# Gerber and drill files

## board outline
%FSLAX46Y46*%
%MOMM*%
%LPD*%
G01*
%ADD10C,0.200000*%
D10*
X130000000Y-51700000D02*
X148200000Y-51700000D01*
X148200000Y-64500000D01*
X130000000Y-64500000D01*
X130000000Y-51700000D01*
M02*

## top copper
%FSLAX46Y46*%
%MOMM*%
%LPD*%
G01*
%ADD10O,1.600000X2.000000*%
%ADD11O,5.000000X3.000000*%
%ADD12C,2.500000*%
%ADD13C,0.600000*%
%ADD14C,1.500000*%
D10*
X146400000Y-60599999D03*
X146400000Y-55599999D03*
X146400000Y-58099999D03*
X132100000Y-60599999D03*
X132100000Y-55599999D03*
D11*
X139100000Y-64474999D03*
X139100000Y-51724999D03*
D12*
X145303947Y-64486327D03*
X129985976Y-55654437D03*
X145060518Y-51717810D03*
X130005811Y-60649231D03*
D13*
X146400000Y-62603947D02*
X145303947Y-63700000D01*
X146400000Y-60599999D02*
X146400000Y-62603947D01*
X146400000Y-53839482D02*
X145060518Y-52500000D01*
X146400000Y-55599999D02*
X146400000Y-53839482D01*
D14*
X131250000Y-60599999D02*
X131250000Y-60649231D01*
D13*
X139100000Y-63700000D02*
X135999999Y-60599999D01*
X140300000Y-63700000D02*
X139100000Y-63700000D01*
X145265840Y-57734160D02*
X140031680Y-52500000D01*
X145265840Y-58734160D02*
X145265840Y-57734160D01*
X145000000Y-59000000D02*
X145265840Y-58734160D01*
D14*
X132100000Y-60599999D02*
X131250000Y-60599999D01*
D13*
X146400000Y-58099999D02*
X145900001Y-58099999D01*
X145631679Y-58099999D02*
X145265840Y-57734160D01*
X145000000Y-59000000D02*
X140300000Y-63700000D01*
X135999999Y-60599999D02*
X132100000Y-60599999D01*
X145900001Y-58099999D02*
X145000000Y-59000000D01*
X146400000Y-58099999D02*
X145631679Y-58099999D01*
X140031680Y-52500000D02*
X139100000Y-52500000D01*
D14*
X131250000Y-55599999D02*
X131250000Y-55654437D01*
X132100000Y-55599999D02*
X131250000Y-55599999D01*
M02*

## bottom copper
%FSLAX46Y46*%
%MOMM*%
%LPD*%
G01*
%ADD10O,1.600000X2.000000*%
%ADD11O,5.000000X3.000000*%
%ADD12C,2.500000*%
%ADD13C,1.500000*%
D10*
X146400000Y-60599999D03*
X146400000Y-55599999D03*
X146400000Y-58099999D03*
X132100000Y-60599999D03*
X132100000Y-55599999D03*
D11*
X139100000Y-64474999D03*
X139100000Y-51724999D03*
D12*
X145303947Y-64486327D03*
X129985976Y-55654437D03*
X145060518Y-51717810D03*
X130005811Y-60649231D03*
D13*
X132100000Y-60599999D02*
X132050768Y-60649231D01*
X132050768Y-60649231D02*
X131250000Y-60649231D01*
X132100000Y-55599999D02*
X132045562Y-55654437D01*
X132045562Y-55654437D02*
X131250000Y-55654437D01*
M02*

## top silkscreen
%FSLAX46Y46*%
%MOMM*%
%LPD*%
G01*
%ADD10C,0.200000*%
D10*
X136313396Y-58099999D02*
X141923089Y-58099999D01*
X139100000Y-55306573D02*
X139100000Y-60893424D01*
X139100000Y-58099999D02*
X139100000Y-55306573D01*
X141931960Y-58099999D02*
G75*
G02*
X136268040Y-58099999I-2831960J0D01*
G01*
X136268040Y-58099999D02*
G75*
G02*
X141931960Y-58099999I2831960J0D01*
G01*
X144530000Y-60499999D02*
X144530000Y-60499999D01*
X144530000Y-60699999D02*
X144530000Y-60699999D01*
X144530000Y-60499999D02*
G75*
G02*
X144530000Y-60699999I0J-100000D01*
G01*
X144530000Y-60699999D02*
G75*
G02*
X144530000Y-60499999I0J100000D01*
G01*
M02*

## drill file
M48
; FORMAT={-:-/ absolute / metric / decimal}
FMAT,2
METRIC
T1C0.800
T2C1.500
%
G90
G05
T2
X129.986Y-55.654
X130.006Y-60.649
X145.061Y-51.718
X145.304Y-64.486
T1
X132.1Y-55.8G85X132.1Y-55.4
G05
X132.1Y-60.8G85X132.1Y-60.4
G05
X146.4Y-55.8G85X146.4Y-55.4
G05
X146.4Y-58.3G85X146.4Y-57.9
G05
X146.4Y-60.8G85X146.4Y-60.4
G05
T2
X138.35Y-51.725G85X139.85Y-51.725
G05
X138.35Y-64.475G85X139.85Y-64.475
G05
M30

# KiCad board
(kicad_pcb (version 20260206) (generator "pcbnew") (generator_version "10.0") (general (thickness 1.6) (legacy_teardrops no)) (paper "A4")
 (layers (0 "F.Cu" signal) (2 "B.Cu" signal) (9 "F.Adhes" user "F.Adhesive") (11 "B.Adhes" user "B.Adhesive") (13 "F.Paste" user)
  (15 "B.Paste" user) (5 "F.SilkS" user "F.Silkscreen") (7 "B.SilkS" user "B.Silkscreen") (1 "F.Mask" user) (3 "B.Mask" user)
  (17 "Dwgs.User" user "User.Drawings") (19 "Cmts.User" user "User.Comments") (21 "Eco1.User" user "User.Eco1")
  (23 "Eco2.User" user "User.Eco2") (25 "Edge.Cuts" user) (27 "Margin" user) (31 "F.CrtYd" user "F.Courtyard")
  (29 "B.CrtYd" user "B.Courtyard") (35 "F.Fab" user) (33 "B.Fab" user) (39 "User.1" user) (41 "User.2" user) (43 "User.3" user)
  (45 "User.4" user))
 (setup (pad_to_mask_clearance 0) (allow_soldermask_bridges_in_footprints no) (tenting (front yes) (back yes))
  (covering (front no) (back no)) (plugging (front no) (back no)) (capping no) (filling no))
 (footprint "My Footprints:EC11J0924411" (layer "F.Cu") (at 139.1 58.099999 90)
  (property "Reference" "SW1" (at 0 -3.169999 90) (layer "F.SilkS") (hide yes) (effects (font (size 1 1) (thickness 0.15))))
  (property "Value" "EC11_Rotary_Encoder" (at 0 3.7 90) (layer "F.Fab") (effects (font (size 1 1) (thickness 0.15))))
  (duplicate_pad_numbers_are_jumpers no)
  (fp_line (start -2.4 5.43) (end -2.4 5.43) (stroke (width 0.2) (type solid)) (layer "F.SilkS"))
  (fp_line (start -2.6 5.43) (end -2.6 5.43) (stroke (width 0.2) (type solid)) (layer "F.SilkS"))
  (fp_arc (start -2.4 5.43) (mid -2.5 5.53) (end -2.6 5.43) (stroke (width 0.2) (type solid)) (layer "F.SilkS"))
  (fp_arc (start -2.6 5.43) (mid -2.5 5.33) (end -2.4 5.43) (stroke (width 0.2) (type solid)) (layer "F.SilkS"))
  (pad "A" thru_hole oval (at -2.5 7.3 90) (size 2 1.6) (drill oval 1.2 0.8) (layers "*.Cu" "*.Mask") (remove_unused_layers no)
   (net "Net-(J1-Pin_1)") (solder_mask_margin 0.102))
  (pad "B" thru_hole oval (at 2.5 7.3 90) (size 2 1.6) (drill oval 1.2 0.8) (layers "*.Cu" "*.Mask") (remove_unused_layers no)
   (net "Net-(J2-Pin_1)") (solder_mask_margin 0.102))
  (pad "C" thru_hole oval (at 0 7.3 90) (size 2 1.6) (drill oval 1.2 0.8) (layers "*.Cu" "*.Mask") (remove_unused_layers no) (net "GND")
   (solder_mask_margin 0.102))
  (pad "D" thru_hole oval (at -2.5 -7 90) (size 2 1.6) (drill oval 1.2 0.8) (layers "*.Cu" "*.Mask") (remove_unused_layers no) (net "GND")
   (solder_mask_margin 0.102))
  (pad "E" thru_hole oval (at 2.5 -7 90) (size 2 1.6) (drill oval 1.2 0.8) (layers "*.Cu" "*.Mask") (remove_unused_layers no)
   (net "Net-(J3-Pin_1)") (solder_mask_margin 0.102))
  (pad "G" thru_hole oval (at -6.375 0 90) (size 3 5) (drill oval 1.5 3) (layers "*.Cu" "*.Mask") (remove_unused_layers no) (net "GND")
   (solder_mask_margin 0.102))
  (pad "G" thru_hole oval (at 6.375 0 90) (size 3 5) (drill oval 1.5 3) (layers "*.Cu" "*.Mask") (remove_unused_layers no) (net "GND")
   (solder_mask_margin 0.102)))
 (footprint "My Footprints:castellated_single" (layer "F.Cu") (at 145.303947 64.486327)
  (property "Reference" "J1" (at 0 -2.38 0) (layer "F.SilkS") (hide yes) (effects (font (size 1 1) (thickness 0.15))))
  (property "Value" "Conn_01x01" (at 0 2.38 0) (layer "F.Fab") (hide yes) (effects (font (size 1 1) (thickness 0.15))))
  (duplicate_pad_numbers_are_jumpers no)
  (pad "1" thru_hole circle (at 0 0) (size 2.5 2.5) (drill 1.5) (layers "*.Cu" "*.Mask") (remove_unused_layers no) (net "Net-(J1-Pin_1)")))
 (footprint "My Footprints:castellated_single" (layer "F.Cu") (at 129.985976 55.654437 -90)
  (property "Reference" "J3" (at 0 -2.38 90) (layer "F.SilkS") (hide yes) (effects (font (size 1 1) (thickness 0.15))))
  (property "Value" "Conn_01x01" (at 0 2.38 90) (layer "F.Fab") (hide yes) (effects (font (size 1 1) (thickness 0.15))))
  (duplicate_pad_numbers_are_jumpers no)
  (pad "1" thru_hole circle (at 0 0 270) (size 2.5 2.5) (drill 1.5) (layers "*.Cu" "*.Mask") (remove_unused_layers no)
   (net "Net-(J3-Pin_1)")))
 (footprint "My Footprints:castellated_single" (layer "F.Cu") (at 145.060518 51.71781 180)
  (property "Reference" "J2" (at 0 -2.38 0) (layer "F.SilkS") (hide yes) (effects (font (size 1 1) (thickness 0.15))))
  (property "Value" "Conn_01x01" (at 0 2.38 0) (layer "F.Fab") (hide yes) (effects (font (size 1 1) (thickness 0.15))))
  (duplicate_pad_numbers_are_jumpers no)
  (pad "1" thru_hole circle (at 0 0 180) (size 2.5 2.5) (drill 1.5) (layers "*.Cu" "*.Mask") (remove_unused_layers no)
   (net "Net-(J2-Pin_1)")))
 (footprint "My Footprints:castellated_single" (layer "F.Cu") (at 130.005811 60.649231 -90)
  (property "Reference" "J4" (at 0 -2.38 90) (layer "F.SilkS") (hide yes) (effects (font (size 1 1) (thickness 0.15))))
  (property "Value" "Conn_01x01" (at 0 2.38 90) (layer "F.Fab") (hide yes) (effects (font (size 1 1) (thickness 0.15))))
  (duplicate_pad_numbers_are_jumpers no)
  (pad "1" thru_hole circle (at 0 0 270) (size 2.5 2.5) (drill 1.5) (layers "*.Cu" "*.Mask") (remove_unused_layers no) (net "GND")))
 (gr_line (start 136.313396 58.099999) (end 141.923089 58.099999) (stroke (width 0.2) (type default)) (layer "F.SilkS"))
 (gr_line (start 139.1 55.306573) (end 139.1 60.893424) (stroke (width 0.2) (type default)) (layer "F.SilkS"))
 (gr_line (start 139.1 58.099999) (end 139.1 55.306573) (stroke (width 0.2) (type default)) (layer "F.SilkS"))
 (gr_circle (center 139.1 58.099999) (end 141 56) (stroke (width 0.2) (type solid)) (fill no) (layer "F.SilkS"))
 (gr_rect (start 130 51.7) (end 148.2 64.5) (stroke (width 0.2) (type solid)) (fill no) (layer "Edge.Cuts"))
 (segment (start 146.4 62.603947) (end 145.303947 63.7) (width 0.6) (layer "F.Cu") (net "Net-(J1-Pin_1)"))
 (segment (start 146.4 60.599999) (end 146.4 62.603947) (width 0.6) (layer "F.Cu") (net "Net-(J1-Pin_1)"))
 (segment (start 146.4 53.839482) (end 145.060518 52.5) (width 0.6) (layer "F.Cu") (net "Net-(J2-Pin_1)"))
 (segment (start 146.4 55.599999) (end 146.4 53.839482) (width 0.6) (layer "F.Cu") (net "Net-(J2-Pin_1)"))
 (segment (start 131.25 60.599999) (end 131.25 60.649231) (width 1.5) (layer "F.Cu") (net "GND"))
 (segment (start 139.1 63.7) (end 135.999999 60.599999) (width 0.6) (layer "F.Cu") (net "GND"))
 (segment (start 140.3 63.7) (end 139.1 63.7) (width 0.6) (layer "F.Cu") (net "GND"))
 (segment (start 145.26584 57.73416) (end 140.03168 52.5) (width 0.6) (layer "F.Cu") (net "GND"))
 (segment (start 145.26584 58.73416) (end 145.26584 57.73416) (width 0.6) (layer "F.Cu") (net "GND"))
 (segment (start 145 59) (end 145.26584 58.73416) (width 0.6) (layer "F.Cu") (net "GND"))
 (segment (start 132.1 60.599999) (end 131.25 60.599999) (width 1.5) (layer "F.Cu") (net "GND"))
 (segment (start 146.4 58.099999) (end 145.900001 58.099999) (width 0.6) (layer "F.Cu") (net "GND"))
 (segment (start 145.631679 58.099999) (end 145.26584 57.73416) (width 0.6) (layer "F.Cu") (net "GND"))
 (segment (start 145 59) (end 140.3 63.7) (width 0.6) (layer "F.Cu") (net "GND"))
 (segment (start 135.999999 60.599999) (end 132.1 60.599999) (width 0.6) (layer "F.Cu") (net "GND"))
 (segment (start 145.900001 58.099999) (end 145 59) (width 0.6) (layer "F.Cu") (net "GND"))
 (segment (start 146.4 58.099999) (end 145.631679 58.099999) (width 0.6) (layer "F.Cu") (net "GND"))
 (segment (start 140.03168 52.5) (end 139.1 52.5) (width 0.6) (layer "F.Cu") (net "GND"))
 (segment (start 132.1 60.599999) (end 132.050768 60.649231) (width 1.5) (layer "B.Cu") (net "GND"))
 (segment (start 132.050768 60.649231) (end 131.25 60.649231) (width 1.5) (layer "B.Cu") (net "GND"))
 (segment (start 131.25 55.599999) (end 131.25 55.654437) (width 1.5) (layer "F.Cu") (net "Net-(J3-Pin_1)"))
 (segment (start 132.1 55.599999) (end 131.25 55.599999) (width 1.5) (layer "F.Cu") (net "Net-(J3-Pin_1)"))
 (segment (start 132.1 55.599999) (end 132.045562 55.654437) (width 1.5) (layer "B.Cu") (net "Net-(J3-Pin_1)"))
 (segment (start 132.045562 55.654437) (end 131.25 55.654437) (width 1.5) (layer "B.Cu") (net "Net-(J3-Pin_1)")))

